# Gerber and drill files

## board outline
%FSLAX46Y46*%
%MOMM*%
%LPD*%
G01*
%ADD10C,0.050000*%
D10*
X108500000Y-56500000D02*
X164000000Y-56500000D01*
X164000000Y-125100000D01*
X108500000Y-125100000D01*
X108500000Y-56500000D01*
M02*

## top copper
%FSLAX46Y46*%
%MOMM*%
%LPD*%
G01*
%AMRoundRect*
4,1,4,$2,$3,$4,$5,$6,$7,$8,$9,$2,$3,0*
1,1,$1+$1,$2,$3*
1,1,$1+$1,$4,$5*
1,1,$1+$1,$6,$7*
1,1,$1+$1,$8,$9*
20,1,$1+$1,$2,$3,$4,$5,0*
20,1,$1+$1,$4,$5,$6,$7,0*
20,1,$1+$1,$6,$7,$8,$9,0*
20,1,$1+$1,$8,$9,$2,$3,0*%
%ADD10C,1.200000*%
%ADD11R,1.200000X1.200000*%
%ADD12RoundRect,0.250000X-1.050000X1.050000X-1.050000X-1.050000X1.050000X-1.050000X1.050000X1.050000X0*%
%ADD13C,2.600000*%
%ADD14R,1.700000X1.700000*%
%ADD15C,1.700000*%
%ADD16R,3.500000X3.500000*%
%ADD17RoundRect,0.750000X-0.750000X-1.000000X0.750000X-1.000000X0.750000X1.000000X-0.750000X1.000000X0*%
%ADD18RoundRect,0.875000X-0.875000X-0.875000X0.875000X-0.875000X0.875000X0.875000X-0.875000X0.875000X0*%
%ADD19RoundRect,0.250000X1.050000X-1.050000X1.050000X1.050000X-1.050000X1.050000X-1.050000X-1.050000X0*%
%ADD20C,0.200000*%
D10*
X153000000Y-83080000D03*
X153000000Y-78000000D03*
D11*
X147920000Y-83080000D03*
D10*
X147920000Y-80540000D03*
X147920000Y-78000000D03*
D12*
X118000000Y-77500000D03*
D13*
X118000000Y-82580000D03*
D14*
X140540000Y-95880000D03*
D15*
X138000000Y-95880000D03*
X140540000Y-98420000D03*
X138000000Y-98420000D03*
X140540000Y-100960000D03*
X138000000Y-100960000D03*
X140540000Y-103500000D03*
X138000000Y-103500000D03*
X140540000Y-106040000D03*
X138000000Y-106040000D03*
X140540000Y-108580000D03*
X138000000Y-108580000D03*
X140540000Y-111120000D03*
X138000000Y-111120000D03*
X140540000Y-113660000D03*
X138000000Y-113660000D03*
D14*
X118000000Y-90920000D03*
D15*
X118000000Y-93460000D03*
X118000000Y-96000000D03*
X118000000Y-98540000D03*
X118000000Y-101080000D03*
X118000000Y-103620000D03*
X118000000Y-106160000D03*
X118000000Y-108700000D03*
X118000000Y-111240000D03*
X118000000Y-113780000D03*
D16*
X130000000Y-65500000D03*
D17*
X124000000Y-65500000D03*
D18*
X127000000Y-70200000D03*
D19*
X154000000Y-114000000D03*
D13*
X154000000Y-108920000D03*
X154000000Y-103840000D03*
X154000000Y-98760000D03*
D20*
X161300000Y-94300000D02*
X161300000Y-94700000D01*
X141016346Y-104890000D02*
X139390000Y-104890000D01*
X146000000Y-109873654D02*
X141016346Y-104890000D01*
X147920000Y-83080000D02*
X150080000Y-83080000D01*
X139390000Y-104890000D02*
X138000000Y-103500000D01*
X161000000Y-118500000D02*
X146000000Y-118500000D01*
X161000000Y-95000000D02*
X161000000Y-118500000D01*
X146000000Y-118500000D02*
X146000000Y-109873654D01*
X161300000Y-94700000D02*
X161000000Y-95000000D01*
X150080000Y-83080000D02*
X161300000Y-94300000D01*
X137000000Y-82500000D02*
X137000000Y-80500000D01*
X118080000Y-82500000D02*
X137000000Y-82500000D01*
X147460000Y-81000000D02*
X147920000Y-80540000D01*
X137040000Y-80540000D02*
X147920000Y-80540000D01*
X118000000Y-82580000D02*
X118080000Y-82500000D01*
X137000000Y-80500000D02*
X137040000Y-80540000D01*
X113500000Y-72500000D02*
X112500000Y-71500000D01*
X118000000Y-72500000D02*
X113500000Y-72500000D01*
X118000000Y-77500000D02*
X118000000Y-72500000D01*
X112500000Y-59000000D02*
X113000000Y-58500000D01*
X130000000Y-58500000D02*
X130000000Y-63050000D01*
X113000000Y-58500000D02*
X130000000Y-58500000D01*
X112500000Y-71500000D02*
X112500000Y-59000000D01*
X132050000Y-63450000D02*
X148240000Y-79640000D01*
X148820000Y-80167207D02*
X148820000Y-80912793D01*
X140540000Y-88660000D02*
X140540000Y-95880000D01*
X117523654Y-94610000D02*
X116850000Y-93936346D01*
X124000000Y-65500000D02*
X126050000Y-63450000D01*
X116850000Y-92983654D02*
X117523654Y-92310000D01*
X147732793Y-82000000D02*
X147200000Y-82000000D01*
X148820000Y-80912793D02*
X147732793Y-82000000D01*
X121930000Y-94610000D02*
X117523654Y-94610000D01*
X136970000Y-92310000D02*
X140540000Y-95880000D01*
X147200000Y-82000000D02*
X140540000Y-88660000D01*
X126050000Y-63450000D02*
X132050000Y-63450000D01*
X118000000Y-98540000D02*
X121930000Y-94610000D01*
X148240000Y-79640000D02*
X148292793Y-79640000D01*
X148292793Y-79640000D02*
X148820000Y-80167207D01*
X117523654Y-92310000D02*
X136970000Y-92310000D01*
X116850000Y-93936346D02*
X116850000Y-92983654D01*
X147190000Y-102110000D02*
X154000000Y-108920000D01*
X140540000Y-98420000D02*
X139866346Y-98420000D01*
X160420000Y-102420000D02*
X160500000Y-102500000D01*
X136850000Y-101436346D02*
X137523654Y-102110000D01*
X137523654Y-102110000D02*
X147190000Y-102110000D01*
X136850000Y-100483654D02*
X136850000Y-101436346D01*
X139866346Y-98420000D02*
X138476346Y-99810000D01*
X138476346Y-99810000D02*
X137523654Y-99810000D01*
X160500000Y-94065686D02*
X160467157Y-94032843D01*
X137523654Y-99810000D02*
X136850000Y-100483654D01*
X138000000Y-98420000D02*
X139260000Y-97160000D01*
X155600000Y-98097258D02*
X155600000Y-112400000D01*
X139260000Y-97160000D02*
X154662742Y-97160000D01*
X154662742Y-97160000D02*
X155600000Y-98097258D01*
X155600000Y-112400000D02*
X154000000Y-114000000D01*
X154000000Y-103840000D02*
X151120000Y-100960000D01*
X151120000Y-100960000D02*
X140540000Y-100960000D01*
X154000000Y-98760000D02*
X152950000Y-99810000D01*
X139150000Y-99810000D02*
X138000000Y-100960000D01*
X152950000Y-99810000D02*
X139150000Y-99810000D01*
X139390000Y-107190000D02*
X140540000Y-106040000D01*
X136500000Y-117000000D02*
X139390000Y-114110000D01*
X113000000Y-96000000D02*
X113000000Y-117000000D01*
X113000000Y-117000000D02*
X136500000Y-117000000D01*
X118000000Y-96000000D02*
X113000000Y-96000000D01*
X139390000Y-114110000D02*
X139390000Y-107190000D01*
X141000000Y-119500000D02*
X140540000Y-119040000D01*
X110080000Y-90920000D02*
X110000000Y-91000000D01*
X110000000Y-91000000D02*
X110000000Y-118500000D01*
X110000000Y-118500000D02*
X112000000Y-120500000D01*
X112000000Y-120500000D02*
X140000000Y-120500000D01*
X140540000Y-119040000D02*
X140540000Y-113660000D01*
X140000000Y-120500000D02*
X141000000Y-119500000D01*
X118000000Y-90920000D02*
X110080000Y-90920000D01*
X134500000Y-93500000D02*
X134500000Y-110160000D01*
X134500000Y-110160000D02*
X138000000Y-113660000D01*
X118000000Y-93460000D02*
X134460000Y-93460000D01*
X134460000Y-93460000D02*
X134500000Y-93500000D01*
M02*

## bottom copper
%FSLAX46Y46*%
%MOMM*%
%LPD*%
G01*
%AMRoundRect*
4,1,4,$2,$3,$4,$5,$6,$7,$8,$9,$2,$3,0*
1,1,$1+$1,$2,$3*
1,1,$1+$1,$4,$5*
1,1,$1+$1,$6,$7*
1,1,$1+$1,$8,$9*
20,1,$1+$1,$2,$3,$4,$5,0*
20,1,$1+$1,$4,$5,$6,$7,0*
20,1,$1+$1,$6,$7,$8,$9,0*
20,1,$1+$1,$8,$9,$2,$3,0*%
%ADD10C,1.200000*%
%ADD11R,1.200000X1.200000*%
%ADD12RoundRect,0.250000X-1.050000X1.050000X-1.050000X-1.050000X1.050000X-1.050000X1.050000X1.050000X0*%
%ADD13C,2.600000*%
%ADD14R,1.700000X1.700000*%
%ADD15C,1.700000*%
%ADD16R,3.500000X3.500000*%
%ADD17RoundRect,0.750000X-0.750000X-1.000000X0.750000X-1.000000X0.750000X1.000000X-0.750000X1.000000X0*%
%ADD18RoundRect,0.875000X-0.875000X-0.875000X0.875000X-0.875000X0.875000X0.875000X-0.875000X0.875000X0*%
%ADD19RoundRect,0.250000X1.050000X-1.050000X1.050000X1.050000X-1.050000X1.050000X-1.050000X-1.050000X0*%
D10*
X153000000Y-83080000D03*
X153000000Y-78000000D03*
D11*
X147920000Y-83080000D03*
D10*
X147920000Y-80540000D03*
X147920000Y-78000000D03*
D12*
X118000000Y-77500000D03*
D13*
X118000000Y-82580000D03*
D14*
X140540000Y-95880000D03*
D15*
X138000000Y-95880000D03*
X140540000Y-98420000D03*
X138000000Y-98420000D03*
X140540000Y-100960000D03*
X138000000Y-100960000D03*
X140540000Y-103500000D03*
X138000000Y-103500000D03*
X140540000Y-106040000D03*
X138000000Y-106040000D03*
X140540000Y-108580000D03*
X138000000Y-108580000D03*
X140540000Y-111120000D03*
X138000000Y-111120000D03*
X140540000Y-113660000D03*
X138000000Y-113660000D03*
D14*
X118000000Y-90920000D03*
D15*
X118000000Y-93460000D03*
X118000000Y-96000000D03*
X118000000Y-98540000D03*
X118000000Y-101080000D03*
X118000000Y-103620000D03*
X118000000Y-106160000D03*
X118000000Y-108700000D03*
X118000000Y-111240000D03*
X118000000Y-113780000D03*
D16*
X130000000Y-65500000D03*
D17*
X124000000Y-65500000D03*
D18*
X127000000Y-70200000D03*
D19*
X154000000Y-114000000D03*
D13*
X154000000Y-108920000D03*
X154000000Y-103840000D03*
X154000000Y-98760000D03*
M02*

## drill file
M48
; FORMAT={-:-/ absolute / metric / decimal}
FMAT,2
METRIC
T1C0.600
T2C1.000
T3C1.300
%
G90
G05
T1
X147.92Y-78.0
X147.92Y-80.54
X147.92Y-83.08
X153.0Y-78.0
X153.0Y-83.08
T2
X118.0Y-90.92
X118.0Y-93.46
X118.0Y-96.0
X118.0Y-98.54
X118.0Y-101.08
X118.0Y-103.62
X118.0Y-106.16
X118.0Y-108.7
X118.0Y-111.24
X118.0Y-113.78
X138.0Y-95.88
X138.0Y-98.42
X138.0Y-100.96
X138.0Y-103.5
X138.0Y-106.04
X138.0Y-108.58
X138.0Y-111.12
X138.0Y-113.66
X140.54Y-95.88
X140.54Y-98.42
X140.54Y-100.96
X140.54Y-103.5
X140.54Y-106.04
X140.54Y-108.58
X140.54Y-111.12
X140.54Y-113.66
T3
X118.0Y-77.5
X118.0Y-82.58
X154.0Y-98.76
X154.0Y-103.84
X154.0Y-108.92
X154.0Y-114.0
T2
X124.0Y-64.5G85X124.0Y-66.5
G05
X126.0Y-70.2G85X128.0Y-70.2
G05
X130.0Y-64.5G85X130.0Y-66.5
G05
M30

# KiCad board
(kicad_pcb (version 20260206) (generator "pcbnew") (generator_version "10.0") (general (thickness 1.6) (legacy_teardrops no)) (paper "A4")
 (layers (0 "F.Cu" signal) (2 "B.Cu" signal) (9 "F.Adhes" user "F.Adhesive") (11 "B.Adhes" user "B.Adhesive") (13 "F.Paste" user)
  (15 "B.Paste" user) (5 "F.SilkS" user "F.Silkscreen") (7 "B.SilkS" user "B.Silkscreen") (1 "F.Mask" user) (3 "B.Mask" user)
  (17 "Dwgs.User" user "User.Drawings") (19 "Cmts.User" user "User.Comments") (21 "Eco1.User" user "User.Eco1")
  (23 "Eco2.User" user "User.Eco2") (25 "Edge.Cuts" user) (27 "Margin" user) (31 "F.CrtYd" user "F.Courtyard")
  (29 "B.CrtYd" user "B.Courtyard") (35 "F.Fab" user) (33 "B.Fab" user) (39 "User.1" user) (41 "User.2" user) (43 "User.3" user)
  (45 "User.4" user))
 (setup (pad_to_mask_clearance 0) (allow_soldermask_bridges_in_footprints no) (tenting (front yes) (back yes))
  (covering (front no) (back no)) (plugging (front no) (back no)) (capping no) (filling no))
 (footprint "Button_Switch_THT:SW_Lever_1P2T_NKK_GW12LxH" (layer "F.Cu") (at 147.92 83.08 90)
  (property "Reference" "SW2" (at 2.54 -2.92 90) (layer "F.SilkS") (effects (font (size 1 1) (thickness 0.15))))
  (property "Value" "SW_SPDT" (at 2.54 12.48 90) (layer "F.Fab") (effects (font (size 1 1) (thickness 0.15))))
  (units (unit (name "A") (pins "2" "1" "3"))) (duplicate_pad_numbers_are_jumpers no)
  (pad "" thru_hole circle (at 0 5.08 90) (size 1.2 1.2) (drill 0.6) (layers "*.Cu" "*.Mask") (remove_unused_layers no))
  (pad "" thru_hole circle (at 5.08 5.08 90) (size 1.2 1.2) (drill 0.6) (layers "*.Cu" "*.Mask") (remove_unused_layers no))
  (pad "1" thru_hole rect (at 0 0 90) (size 1.2 1.2) (drill 0.6) (layers "*.Cu" "*.Mask") (remove_unused_layers no) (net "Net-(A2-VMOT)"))
  (pad "2" thru_hole circle (at 2.54 0 90) (size 1.2 1.2) (drill 0.6) (layers "*.Cu" "*.Mask") (remove_unused_layers no) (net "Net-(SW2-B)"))
  (pad "3" thru_hole circle (at 5.08 0 90) (size 1.2 1.2) (drill 0.6) (layers "*.Cu" "*.Mask") (remove_unused_layers no)
   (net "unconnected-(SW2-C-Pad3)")))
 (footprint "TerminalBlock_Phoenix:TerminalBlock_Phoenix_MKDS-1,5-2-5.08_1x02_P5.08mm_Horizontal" (layer "F.Cu") (at 118 77.5 -90)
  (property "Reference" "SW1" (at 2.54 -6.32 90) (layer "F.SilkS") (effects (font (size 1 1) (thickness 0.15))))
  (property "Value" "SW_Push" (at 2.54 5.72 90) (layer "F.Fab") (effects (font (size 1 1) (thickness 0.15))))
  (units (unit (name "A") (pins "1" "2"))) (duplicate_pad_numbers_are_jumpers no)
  (pad "1" thru_hole roundrect (at 0 0 270) (size 2.6 2.6) (drill 1.3) (layers "*.Cu" "*.Mask") (remove_unused_layers no)
   (roundrect_rratio 0.096154) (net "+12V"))
  (pad "2" thru_hole circle (at 5.08 0 270) (size 2.6 2.6) (drill 1.3) (layers "*.Cu" "*.Mask") (remove_unused_layers no)
   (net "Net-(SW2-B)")))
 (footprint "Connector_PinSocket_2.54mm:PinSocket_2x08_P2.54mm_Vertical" (layer "F.Cu") (at 140.54 95.88)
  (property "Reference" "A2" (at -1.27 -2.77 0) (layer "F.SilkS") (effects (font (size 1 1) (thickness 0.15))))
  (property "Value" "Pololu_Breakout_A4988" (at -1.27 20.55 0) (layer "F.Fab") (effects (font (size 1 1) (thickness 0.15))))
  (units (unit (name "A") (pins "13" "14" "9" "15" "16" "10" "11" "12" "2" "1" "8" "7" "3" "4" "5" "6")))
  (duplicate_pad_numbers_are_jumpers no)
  (pad "1" thru_hole rect (at 0 0) (size 1.7 1.7) (drill 1) (layers "*.Cu" "*.Mask") (remove_unused_layers no) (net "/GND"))
  (pad "2" thru_hole circle (at -2.54 0) (size 1.7 1.7) (drill 1) (layers "*.Cu" "*.Mask") (remove_unused_layers no)
   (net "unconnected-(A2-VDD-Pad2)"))
  (pad "3" thru_hole circle (at 0 2.54) (size 1.7 1.7) (drill 1) (layers "*.Cu" "*.Mask") (remove_unused_layers no) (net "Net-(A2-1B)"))
  (pad "4" thru_hole circle (at -2.54 2.54) (size 1.7 1.7) (drill 1) (layers "*.Cu" "*.Mask") (remove_unused_layers no) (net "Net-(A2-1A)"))
  (pad "5" thru_hole circle (at 0 5.08) (size 1.7 1.7) (drill 1) (layers "*.Cu" "*.Mask") (remove_unused_layers no) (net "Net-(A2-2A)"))
  (pad "6" thru_hole circle (at -2.54 5.08) (size 1.7 1.7) (drill 1) (layers "*.Cu" "*.Mask") (remove_unused_layers no) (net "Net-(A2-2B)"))
  (pad "7" thru_hole circle (at 0 7.62) (size 1.7 1.7) (drill 1) (layers "*.Cu" "*.Mask") (remove_unused_layers no)
   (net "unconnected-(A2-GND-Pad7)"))
  (pad "8" thru_hole circle (at -2.54 7.62) (size 1.7 1.7) (drill 1) (layers "*.Cu" "*.Mask") (remove_unused_layers no)
   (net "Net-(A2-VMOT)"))
  (pad "9" thru_hole circle (at 0 10.16) (size 1.7 1.7) (drill 1) (layers "*.Cu" "*.Mask") (remove_unused_layers no) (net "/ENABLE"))
  (pad "10" thru_hole circle (at -2.54 10.16) (size 1.7 1.7) (drill 1) (layers "*.Cu" "*.Mask") (remove_unused_layers no)
   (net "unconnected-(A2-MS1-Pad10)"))
  (pad "11" thru_hole circle (at 0 12.7) (size 1.7 1.7) (drill 1) (layers "*.Cu" "*.Mask") (remove_unused_layers no)
   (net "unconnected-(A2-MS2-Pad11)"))
  (pad "12" thru_hole circle (at -2.54 12.7) (size 1.7 1.7) (drill 1) (layers "*.Cu" "*.Mask") (remove_unused_layers no)
   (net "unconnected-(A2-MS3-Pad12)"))
  (pad "13" thru_hole circle (at 0 15.24) (size 1.7 1.7) (drill 1) (layers "*.Cu" "*.Mask") (remove_unused_layers no)
   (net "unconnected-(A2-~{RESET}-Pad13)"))
  (pad "14" thru_hole circle (at -2.54 15.24) (size 1.7 1.7) (drill 1) (layers "*.Cu" "*.Mask") (remove_unused_layers no)
   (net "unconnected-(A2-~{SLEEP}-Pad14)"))
  (pad "15" thru_hole circle (at 0 17.78) (size 1.7 1.7) (drill 1) (layers "*.Cu" "*.Mask") (remove_unused_layers no) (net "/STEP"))
  (pad "16" thru_hole circle (at -2.54 17.78) (size 1.7 1.7) (drill 1) (layers "*.Cu" "*.Mask") (remove_unused_layers no) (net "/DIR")))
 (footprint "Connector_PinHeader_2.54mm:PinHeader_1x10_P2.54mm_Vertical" (layer "F.Cu") (at 118 90.92)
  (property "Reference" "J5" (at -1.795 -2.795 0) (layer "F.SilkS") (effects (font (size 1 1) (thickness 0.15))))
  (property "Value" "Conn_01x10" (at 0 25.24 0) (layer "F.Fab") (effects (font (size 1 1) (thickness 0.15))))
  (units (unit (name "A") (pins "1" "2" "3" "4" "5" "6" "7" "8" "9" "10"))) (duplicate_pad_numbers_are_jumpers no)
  (pad "1" thru_hole rect (at 0 0) (size 1.7 1.7) (drill 1) (layers "*.Cu" "*.Mask") (remove_unused_layers no) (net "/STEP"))
  (pad "2" thru_hole circle (at 0 2.54) (size 1.7 1.7) (drill 1) (layers "*.Cu" "*.Mask") (remove_unused_layers no) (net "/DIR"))
  (pad "3" thru_hole circle (at 0 5.08) (size 1.7 1.7) (drill 1) (layers "*.Cu" "*.Mask") (remove_unused_layers no) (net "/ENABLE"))
  (pad "4" thru_hole circle (at 0 7.62) (size 1.7 1.7) (drill 1) (layers "*.Cu" "*.Mask") (remove_unused_layers no) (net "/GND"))
  (pad "5" thru_hole circle (at 0 10.16) (size 1.7 1.7) (drill 1) (layers "*.Cu" "*.Mask") (remove_unused_layers no)
   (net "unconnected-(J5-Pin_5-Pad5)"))
  (pad "6" thru_hole circle (at 0 12.7) (size 1.7 1.7) (drill 1) (layers "*.Cu" "*.Mask") (remove_unused_layers no)
   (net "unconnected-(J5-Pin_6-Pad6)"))
  (pad "7" thru_hole circle (at 0 15.24) (size 1.7 1.7) (drill 1) (layers "*.Cu" "*.Mask") (remove_unused_layers no)
   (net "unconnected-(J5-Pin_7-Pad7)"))
  (pad "8" thru_hole circle (at 0 17.78) (size 1.7 1.7) (drill 1) (layers "*.Cu" "*.Mask") (remove_unused_layers no)
   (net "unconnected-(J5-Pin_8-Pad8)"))
  (pad "9" thru_hole circle (at 0 20.32) (size 1.7 1.7) (drill 1) (layers "*.Cu" "*.Mask") (remove_unused_layers no)
   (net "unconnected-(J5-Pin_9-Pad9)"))
  (pad "10" thru_hole circle (at 0 22.86) (size 1.7 1.7) (drill 1) (layers "*.Cu" "*.Mask") (remove_unused_layers no)
   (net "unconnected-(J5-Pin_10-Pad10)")))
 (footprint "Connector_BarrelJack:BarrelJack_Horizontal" (layer "F.Cu") (at 130 65.5)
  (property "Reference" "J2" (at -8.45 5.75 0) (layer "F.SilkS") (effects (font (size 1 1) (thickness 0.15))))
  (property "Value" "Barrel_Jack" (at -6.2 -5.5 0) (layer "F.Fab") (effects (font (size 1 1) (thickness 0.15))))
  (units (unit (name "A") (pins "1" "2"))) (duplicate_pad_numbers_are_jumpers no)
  (pad "1" thru_hole rect (at 0 0) (size 3.5 3.5) (drill oval 1 3) (layers "*.Cu" "*.Mask") (remove_unused_layers no) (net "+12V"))
  (pad "2" thru_hole roundrect (at -6 0) (size 3 3.5) (drill oval 1 3) (layers "*.Cu" "*.Mask") (remove_unused_layers no)
   (roundrect_rratio 0.25) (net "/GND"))
  (pad "3" thru_hole roundrect (at -3 4.7) (size 3.5 3.5) (drill oval 3 1) (layers "*.Cu" "*.Mask") (remove_unused_layers no)
   (roundrect_rratio 0.25)))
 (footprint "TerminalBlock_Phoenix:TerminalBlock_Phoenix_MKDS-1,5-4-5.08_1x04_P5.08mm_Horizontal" (layer "F.Cu") (at 154 114 90)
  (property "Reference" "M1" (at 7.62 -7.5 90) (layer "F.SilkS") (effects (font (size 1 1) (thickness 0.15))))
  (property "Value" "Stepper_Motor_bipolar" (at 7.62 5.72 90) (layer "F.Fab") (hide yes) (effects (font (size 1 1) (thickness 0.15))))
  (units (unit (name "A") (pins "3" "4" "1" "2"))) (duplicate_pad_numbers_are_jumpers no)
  (pad "1" thru_hole roundrect (at 0 0 90) (size 2.6 2.6) (drill 1.3) (layers "*.Cu" "*.Mask") (remove_unused_layers no)
   (roundrect_rratio 0.096154) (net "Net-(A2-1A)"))
  (pad "2" thru_hole circle (at 5.08 0 90) (size 2.6 2.6) (drill 1.3) (layers "*.Cu" "*.Mask") (remove_unused_layers no) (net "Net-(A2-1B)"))
  (pad "3" thru_hole circle (at 10.16 0 90) (size 2.6 2.6) (drill 1.3) (layers "*.Cu" "*.Mask") (remove_unused_layers no)
   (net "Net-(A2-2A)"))
  (pad "4" thru_hole circle (at 15.24 0 90) (size 2.6 2.6) (drill 1.3) (layers "*.Cu" "*.Mask") (remove_unused_layers no)
   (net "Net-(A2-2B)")))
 (gr_rect (start 108.5 56.5) (end 164 125.1) (stroke (width 0.05) (type default)) (fill no) (layer "Edge.Cuts"))
 (segment (start 161.3 94.3) (end 161.3 94.7) (width 0.2) (layer "F.Cu") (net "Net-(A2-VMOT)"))
 (segment (start 141.016346 104.89) (end 139.39 104.89) (width 0.2) (layer "F.Cu") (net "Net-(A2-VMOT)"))
 (segment (start 146 109.873654) (end 141.016346 104.89) (width 0.2) (layer "F.Cu") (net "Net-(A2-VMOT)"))
 (segment (start 147.92 83.08) (end 150.08 83.08) (width 0.2) (layer "F.Cu") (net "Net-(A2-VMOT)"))
 (segment (start 139.39 104.89) (end 138 103.5) (width 0.2) (layer "F.Cu") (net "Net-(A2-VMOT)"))
 (segment (start 161 118.5) (end 146 118.5) (width 0.2) (layer "F.Cu") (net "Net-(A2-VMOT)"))
 (segment (start 161 95) (end 161 118.5) (width 0.2) (layer "F.Cu") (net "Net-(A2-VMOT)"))
 (segment (start 146 118.5) (end 146 109.873654) (width 0.2) (layer "F.Cu") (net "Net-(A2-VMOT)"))
 (segment (start 161.3 94.7) (end 161 95) (width 0.2) (layer "F.Cu") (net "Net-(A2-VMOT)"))
 (segment (start 150.08 83.08) (end 161.3 94.3) (width 0.2) (layer "F.Cu") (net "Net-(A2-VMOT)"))
 (segment (start 137 82.5) (end 137 80.5) (width 0.2) (layer "F.Cu") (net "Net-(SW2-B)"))
 (segment (start 118.08 82.5) (end 137 82.5) (width 0.2) (layer "F.Cu") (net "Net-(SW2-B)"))
 (segment (start 147.46 81) (end 147.92 80.54) (width 0.2) (layer "F.Cu") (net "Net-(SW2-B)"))
 (segment (start 137.04 80.54) (end 147.92 80.54) (width 0.2) (layer "F.Cu") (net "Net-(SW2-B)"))
 (segment (start 118 82.58) (end 118.08 82.5) (width 0.2) (layer "F.Cu") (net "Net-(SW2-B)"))
 (segment (start 137 80.5) (end 137.04 80.54) (width 0.2) (layer "F.Cu") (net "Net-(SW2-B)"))
 (segment (start 113.5 72.5) (end 112.5 71.5) (width 0.2) (layer "F.Cu") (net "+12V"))
 (segment (start 118 72.5) (end 113.5 72.5) (width 0.2) (layer "F.Cu") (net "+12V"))
 (segment (start 118 77.5) (end 118 72.5) (width 0.2) (layer "F.Cu") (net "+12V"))
 (segment (start 112.5 59) (end 113 58.5) (width 0.2) (layer "F.Cu") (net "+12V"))
 (segment (start 130 58.5) (end 130 63.05) (width 0.2) (layer "F.Cu") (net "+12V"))
 (segment (start 113 58.5) (end 130 58.5) (width 0.2) (layer "F.Cu") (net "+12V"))
 (segment (start 112.5 71.5) (end 112.5 59) (width 0.2) (layer "F.Cu") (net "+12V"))
 (segment (start 132.05 63.45) (end 148.24 79.64) (width 0.2) (layer "F.Cu") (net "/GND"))
 (segment (start 148.82 80.167207) (end 148.82 80.912793) (width 0.2) (layer "F.Cu") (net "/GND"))
 (segment (start 140.54 88.66) (end 140.54 95.88) (width 0.2) (layer "F.Cu") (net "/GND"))
 (segment (start 117.523654 94.61) (end 116.85 93.936346) (width 0.2) (layer "F.Cu") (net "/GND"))
 (segment (start 124 65.5) (end 126.05 63.45) (width 0.2) (layer "F.Cu") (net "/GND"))
 (segment (start 116.85 92.983654) (end 117.523654 92.31) (width 0.2) (layer "F.Cu") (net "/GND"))
 (segment (start 147.732793 82) (end 147.2 82) (width 0.2) (layer "F.Cu") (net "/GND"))
 (segment (start 148.82 80.912793) (end 147.732793 82) (width 0.2) (layer "F.Cu") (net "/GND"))
 (segment (start 121.93 94.61) (end 117.523654 94.61) (width 0.2) (layer "F.Cu") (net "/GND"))
 (segment (start 136.97 92.31) (end 140.54 95.88) (width 0.2) (layer "F.Cu") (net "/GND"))
 (segment (start 147.2 82) (end 140.54 88.66) (width 0.2) (layer "F.Cu") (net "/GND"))
 (segment (start 126.05 63.45) (end 132.05 63.45) (width 0.2) (layer "F.Cu") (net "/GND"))
 (segment (start 118 98.54) (end 121.93 94.61) (width 0.2) (layer "F.Cu") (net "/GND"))
 (segment (start 148.24 79.64) (end 148.292793 79.64) (width 0.2) (layer "F.Cu") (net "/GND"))
 (segment (start 148.292793 79.64) (end 148.82 80.167207) (width 0.2) (layer "F.Cu") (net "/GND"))
 (segment (start 117.523654 92.31) (end 136.97 92.31) (width 0.2) (layer "F.Cu") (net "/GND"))
 (segment (start 116.85 93.936346) (end 116.85 92.983654) (width 0.2) (layer "F.Cu") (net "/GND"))
 (segment (start 147.19 102.11) (end 154 108.92) (width 0.2) (layer "F.Cu") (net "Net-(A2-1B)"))
 (segment (start 140.54 98.42) (end 139.866346 98.42) (width 0.2) (layer "F.Cu") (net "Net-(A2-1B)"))
 (segment (start 160.42 102.42) (end 160.5 102.5) (width 0.2) (layer "F.Cu") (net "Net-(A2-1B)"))
 (segment (start 136.85 101.436346) (end 137.523654 102.11) (width 0.2) (layer "F.Cu") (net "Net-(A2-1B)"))
 (segment (start 137.523654 102.11) (end 147.19 102.11) (width 0.2) (layer "F.Cu") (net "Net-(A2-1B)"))
 (segment (start 136.85 100.483654) (end 136.85 101.436346) (width 0.2) (layer "F.Cu") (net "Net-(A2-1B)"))
 (segment (start 139.866346 98.42) (end 138.476346 99.81) (width 0.2) (layer "F.Cu") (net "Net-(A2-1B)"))
 (segment (start 138.476346 99.81) (end 137.523654 99.81) (width 0.2) (layer "F.Cu") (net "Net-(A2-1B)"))
 (segment (start 160.5 94.065686) (end 160.467157 94.032843) (width 0.2) (layer "F.Cu") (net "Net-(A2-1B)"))
 (segment (start 137.523654 99.81) (end 136.85 100.483654) (width 0.2) (layer "F.Cu") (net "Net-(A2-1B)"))
 (segment (start 138 98.42) (end 139.26 97.16) (width 0.2) (layer "F.Cu") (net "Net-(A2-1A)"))
 (segment (start 155.6 98.097258) (end 155.6 112.4) (width 0.2) (layer "F.Cu") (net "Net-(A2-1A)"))
 (segment (start 139.26 97.16) (end 154.662742 97.16) (width 0.2) (layer "F.Cu") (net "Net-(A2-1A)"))
 (segment (start 154.662742 97.16) (end 155.6 98.097258) (width 0.2) (layer "F.Cu") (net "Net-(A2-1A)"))
 (segment (start 155.6 112.4) (end 154 114) (width 0.2) (layer "F.Cu") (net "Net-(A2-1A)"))
 (segment (start 154 103.84) (end 151.12 100.96) (width 0.2) (layer "F.Cu") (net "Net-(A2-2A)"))
 (segment (start 151.12 100.96) (end 140.54 100.96) (width 0.2) (layer "F.Cu") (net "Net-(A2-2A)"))
 (segment (start 154 98.76) (end 152.95 99.81) (width 0.2) (layer "F.Cu") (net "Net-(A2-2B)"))
 (segment (start 139.15 99.81) (end 138 100.96) (width 0.2) (layer "F.Cu") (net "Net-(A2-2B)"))
 (segment (start 152.95 99.81) (end 139.15 99.81) (width 0.2) (layer "F.Cu") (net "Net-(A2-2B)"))
 (segment (start 139.39 107.19) (end 140.54 106.04) (width 0.2) (layer "F.Cu") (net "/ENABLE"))
 (segment (start 136.5 117) (end 139.39 114.11) (width 0.2) (layer "F.Cu") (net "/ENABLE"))
 (segment (start 113 96) (end 113 117) (width 0.2) (layer "F.Cu") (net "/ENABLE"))
 (segment (start 113 117) (end 136.5 117) (width 0.2) (layer "F.Cu") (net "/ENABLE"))
 (segment (start 118 96) (end 113 96) (width 0.2) (layer "F.Cu") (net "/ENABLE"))
 (segment (start 139.39 114.11) (end 139.39 107.19) (width 0.2) (layer "F.Cu") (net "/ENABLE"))
 (segment (start 141 119.5) (end 140.54 119.04) (width 0.2) (layer "F.Cu") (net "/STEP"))
 (segment (start 110.08 90.92) (end 110 91) (width 0.2) (layer "F.Cu") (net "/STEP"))
 (segment (start 110 91) (end 110 118.5) (width 0.2) (layer "F.Cu") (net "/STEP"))
 (segment (start 110 118.5) (end 112 120.5) (width 0.2) (layer "F.Cu") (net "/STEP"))
 (segment (start 112 120.5) (end 140 120.5) (width 0.2) (layer "F.Cu") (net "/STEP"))
 (segment (start 140.54 119.04) (end 140.54 113.66) (width 0.2) (layer "F.Cu") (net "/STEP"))
 (segment (start 140 120.5) (end 141 119.5) (width 0.2) (layer "F.Cu") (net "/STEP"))
 (segment (start 118 90.92) (end 110.08 90.92) (width 0.2) (layer "F.Cu") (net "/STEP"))
 (segment (start 134.5 93.5) (end 134.5 110.16) (width 0.2) (layer "F.Cu") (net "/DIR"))
 (segment (start 134.5 110.16) (end 138 113.66) (width 0.2) (layer "F.Cu") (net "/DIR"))
 (segment (start 118 93.46) (end 134.46 93.46) (width 0.2) (layer "F.Cu") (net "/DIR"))
 (segment (start 134.46 93.46) (end 134.5 93.5) (width 0.2) (layer "F.Cu") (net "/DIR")))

